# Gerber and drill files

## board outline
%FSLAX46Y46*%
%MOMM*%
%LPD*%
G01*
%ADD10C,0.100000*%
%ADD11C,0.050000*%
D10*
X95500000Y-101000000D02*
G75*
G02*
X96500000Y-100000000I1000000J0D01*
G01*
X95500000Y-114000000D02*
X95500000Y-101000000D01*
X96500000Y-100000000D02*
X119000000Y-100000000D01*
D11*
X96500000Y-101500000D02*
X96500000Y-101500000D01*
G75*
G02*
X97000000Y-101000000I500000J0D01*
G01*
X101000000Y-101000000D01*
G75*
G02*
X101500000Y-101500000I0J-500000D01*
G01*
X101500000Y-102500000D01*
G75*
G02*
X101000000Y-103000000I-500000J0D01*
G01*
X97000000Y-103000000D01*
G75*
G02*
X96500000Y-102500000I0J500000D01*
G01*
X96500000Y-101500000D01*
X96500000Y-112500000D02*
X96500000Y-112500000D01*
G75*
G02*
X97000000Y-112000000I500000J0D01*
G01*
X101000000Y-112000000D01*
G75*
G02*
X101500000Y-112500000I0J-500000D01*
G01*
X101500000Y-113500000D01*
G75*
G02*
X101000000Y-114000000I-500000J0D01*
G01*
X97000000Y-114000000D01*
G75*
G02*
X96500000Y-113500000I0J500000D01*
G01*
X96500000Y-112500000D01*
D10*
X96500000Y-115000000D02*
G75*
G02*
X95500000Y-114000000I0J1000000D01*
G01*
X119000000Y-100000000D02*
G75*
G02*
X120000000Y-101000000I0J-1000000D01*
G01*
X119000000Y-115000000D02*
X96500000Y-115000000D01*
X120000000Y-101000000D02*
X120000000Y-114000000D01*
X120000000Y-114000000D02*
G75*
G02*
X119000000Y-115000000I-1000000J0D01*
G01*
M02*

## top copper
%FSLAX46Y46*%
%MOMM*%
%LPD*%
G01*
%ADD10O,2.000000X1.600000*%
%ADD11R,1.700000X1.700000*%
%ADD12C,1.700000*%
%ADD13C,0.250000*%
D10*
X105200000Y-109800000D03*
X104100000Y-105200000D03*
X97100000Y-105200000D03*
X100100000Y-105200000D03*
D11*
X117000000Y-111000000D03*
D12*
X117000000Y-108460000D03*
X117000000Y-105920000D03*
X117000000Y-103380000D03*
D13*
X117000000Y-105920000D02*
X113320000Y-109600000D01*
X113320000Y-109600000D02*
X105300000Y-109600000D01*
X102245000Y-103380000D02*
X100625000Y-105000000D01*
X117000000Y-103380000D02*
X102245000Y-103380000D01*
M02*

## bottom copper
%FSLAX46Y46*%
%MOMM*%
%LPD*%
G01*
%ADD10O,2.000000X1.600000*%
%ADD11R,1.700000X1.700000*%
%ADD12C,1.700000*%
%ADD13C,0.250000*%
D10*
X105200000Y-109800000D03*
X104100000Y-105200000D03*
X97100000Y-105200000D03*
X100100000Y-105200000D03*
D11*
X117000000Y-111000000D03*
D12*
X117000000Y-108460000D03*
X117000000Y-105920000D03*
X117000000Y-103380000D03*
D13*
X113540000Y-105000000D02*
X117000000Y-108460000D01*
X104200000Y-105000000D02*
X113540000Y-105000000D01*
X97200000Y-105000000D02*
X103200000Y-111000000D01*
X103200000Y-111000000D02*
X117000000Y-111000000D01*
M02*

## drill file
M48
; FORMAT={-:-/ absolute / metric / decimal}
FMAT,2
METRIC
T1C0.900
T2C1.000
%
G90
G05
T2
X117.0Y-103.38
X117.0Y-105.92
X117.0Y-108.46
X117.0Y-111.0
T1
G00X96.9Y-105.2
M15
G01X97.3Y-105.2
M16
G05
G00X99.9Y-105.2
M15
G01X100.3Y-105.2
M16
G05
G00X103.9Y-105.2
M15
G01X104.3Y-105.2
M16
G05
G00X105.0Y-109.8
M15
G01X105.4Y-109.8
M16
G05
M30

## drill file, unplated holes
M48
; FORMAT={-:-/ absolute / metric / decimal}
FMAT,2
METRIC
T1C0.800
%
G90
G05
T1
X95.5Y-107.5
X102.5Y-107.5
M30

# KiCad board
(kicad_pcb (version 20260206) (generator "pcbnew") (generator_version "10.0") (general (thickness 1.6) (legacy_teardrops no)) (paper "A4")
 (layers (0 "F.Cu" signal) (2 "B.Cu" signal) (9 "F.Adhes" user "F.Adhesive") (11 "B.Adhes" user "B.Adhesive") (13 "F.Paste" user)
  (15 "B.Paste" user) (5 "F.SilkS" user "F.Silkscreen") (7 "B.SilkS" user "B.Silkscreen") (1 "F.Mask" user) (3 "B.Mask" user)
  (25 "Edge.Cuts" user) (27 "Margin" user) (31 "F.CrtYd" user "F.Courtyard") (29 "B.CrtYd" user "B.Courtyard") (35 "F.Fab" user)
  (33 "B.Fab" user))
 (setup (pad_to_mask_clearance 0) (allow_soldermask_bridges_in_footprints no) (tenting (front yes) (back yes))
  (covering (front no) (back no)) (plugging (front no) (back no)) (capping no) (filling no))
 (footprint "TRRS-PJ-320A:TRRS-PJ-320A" (layer "F.Cu") (at 93.9 107.5 90)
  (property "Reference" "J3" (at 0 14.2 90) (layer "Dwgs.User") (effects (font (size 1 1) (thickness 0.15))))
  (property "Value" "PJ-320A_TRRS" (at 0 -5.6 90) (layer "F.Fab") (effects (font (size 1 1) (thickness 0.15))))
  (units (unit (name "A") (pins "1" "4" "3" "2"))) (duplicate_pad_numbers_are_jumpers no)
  (pad "" np_thru_hole circle (at 0 1.6 90) (size 0.8 0.8) (drill 0.8) (layers "*.Cu" "*.Mask"))
  (pad "" np_thru_hole circle (at 0 8.6 90) (size 0.8 0.8) (drill 0.8) (layers "*.Cu" "*.Mask"))
  (pad "1" thru_hole oval (at -2.3 11.3 90) (size 1.6 2) (drill oval 0.9 1.3) (layers "*.Cu" "*.Mask") (remove_unused_layers no) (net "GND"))
  (pad "2" thru_hole oval (at 2.3 10.2 90) (size 1.6 2) (drill oval 0.9 1.3) (layers "*.Cu" "*.Mask") (remove_unused_layers no) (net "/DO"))
  (pad "3" thru_hole oval (at 2.3 6.2 90) (size 1.6 2) (drill oval 0.9 1.3) (layers "*.Cu" "*.Mask") (remove_unused_layers no) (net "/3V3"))
  (pad "4" thru_hole oval (at 2.3 3.2 90) (size 1.6 2) (drill oval 0.9 1.3) (layers "*.Cu" "*.Mask") (remove_unused_layers no) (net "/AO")))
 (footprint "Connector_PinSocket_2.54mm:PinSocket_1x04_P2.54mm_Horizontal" (layer "B.Cu") (at 117 111)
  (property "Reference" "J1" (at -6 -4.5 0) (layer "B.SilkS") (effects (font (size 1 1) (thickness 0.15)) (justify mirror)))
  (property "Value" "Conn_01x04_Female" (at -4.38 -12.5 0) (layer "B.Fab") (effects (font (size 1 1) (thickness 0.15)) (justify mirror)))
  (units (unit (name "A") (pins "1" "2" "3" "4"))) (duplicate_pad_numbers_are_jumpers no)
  (pad "1" thru_hole rect (at 0 0) (size 1.7 1.7) (drill 1) (layers "*.Cu" "*.Mask") (remove_unused_layers no) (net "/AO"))
  (pad "2" thru_hole circle (at 0 -2.54) (size 1.7 1.7) (drill 1) (layers "*.Cu" "*.Mask") (remove_unused_layers no) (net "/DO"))
  (pad "3" thru_hole circle (at 0 -5.08) (size 1.7 1.7) (drill 1) (layers "*.Cu" "*.Mask") (remove_unused_layers no) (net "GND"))
  (pad "4" thru_hole circle (at 0 -7.62) (size 1.7 1.7) (drill 1) (layers "*.Cu" "*.Mask") (remove_unused_layers no) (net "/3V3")))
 (gr_arc (start 95.5 101) (mid 95.792893 100.292893) (end 96.5 100) (stroke (width 0.1) (type default)) (layer "Edge.Cuts"))
 (gr_line (start 95.5 114) (end 95.5 101) (stroke (width 0.1) (type default)) (layer "Edge.Cuts"))
 (gr_line (start 96.5 100) (end 119 100) (stroke (width 0.1) (type default)) (layer "Edge.Cuts"))
 (gr_rect (start 96.5 101) (end 101.5 103) (radius 0.5) (stroke (width 0.05) (type solid)) (fill no) (layer "Edge.Cuts"))
 (gr_rect (start 96.5 112) (end 101.5 114) (radius 0.5) (stroke (width 0.05) (type solid)) (fill no) (layer "Edge.Cuts"))
 (gr_arc (start 96.5 115) (mid 95.792893 114.707107) (end 95.5 114) (stroke (width 0.1) (type default)) (layer "Edge.Cuts"))
 (gr_arc (start 119 100) (mid 119.707107 100.292893) (end 120 101) (stroke (width 0.1) (type default)) (layer "Edge.Cuts"))
 (gr_line (start 119 115) (end 96.5 115) (stroke (width 0.1) (type default)) (layer "Edge.Cuts"))
 (gr_line (start 120 101) (end 120 114) (stroke (width 0.1) (type default)) (layer "Edge.Cuts"))
 (gr_arc (start 120 114) (mid 119.707107 114.707107) (end 119 115) (stroke (width 0.1) (type default)) (layer "Edge.Cuts"))
 (segment (start 97.2 105) (end 103.2 111) (width 0.25) (layer "B.Cu") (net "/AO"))
 (segment (start 103.2 111) (end 117 111) (width 0.25) (layer "B.Cu") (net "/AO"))
 (segment (start 113.54 105) (end 117 108.46) (width 0.25) (layer "B.Cu") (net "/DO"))
 (segment (start 104.2 105) (end 113.54 105) (width 0.25) (layer "B.Cu") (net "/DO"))
 (segment (start 117 105.92) (end 113.32 109.6) (width 0.25) (layer "F.Cu") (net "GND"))
 (segment (start 113.32 109.6) (end 105.3 109.6) (width 0.25) (layer "F.Cu") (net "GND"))
 (segment (start 102.245 103.38) (end 100.625 105) (width 0.25) (layer "F.Cu") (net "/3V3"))
 (segment (start 117 103.38) (end 102.245 103.38) (width 0.25) (layer "F.Cu") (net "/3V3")))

